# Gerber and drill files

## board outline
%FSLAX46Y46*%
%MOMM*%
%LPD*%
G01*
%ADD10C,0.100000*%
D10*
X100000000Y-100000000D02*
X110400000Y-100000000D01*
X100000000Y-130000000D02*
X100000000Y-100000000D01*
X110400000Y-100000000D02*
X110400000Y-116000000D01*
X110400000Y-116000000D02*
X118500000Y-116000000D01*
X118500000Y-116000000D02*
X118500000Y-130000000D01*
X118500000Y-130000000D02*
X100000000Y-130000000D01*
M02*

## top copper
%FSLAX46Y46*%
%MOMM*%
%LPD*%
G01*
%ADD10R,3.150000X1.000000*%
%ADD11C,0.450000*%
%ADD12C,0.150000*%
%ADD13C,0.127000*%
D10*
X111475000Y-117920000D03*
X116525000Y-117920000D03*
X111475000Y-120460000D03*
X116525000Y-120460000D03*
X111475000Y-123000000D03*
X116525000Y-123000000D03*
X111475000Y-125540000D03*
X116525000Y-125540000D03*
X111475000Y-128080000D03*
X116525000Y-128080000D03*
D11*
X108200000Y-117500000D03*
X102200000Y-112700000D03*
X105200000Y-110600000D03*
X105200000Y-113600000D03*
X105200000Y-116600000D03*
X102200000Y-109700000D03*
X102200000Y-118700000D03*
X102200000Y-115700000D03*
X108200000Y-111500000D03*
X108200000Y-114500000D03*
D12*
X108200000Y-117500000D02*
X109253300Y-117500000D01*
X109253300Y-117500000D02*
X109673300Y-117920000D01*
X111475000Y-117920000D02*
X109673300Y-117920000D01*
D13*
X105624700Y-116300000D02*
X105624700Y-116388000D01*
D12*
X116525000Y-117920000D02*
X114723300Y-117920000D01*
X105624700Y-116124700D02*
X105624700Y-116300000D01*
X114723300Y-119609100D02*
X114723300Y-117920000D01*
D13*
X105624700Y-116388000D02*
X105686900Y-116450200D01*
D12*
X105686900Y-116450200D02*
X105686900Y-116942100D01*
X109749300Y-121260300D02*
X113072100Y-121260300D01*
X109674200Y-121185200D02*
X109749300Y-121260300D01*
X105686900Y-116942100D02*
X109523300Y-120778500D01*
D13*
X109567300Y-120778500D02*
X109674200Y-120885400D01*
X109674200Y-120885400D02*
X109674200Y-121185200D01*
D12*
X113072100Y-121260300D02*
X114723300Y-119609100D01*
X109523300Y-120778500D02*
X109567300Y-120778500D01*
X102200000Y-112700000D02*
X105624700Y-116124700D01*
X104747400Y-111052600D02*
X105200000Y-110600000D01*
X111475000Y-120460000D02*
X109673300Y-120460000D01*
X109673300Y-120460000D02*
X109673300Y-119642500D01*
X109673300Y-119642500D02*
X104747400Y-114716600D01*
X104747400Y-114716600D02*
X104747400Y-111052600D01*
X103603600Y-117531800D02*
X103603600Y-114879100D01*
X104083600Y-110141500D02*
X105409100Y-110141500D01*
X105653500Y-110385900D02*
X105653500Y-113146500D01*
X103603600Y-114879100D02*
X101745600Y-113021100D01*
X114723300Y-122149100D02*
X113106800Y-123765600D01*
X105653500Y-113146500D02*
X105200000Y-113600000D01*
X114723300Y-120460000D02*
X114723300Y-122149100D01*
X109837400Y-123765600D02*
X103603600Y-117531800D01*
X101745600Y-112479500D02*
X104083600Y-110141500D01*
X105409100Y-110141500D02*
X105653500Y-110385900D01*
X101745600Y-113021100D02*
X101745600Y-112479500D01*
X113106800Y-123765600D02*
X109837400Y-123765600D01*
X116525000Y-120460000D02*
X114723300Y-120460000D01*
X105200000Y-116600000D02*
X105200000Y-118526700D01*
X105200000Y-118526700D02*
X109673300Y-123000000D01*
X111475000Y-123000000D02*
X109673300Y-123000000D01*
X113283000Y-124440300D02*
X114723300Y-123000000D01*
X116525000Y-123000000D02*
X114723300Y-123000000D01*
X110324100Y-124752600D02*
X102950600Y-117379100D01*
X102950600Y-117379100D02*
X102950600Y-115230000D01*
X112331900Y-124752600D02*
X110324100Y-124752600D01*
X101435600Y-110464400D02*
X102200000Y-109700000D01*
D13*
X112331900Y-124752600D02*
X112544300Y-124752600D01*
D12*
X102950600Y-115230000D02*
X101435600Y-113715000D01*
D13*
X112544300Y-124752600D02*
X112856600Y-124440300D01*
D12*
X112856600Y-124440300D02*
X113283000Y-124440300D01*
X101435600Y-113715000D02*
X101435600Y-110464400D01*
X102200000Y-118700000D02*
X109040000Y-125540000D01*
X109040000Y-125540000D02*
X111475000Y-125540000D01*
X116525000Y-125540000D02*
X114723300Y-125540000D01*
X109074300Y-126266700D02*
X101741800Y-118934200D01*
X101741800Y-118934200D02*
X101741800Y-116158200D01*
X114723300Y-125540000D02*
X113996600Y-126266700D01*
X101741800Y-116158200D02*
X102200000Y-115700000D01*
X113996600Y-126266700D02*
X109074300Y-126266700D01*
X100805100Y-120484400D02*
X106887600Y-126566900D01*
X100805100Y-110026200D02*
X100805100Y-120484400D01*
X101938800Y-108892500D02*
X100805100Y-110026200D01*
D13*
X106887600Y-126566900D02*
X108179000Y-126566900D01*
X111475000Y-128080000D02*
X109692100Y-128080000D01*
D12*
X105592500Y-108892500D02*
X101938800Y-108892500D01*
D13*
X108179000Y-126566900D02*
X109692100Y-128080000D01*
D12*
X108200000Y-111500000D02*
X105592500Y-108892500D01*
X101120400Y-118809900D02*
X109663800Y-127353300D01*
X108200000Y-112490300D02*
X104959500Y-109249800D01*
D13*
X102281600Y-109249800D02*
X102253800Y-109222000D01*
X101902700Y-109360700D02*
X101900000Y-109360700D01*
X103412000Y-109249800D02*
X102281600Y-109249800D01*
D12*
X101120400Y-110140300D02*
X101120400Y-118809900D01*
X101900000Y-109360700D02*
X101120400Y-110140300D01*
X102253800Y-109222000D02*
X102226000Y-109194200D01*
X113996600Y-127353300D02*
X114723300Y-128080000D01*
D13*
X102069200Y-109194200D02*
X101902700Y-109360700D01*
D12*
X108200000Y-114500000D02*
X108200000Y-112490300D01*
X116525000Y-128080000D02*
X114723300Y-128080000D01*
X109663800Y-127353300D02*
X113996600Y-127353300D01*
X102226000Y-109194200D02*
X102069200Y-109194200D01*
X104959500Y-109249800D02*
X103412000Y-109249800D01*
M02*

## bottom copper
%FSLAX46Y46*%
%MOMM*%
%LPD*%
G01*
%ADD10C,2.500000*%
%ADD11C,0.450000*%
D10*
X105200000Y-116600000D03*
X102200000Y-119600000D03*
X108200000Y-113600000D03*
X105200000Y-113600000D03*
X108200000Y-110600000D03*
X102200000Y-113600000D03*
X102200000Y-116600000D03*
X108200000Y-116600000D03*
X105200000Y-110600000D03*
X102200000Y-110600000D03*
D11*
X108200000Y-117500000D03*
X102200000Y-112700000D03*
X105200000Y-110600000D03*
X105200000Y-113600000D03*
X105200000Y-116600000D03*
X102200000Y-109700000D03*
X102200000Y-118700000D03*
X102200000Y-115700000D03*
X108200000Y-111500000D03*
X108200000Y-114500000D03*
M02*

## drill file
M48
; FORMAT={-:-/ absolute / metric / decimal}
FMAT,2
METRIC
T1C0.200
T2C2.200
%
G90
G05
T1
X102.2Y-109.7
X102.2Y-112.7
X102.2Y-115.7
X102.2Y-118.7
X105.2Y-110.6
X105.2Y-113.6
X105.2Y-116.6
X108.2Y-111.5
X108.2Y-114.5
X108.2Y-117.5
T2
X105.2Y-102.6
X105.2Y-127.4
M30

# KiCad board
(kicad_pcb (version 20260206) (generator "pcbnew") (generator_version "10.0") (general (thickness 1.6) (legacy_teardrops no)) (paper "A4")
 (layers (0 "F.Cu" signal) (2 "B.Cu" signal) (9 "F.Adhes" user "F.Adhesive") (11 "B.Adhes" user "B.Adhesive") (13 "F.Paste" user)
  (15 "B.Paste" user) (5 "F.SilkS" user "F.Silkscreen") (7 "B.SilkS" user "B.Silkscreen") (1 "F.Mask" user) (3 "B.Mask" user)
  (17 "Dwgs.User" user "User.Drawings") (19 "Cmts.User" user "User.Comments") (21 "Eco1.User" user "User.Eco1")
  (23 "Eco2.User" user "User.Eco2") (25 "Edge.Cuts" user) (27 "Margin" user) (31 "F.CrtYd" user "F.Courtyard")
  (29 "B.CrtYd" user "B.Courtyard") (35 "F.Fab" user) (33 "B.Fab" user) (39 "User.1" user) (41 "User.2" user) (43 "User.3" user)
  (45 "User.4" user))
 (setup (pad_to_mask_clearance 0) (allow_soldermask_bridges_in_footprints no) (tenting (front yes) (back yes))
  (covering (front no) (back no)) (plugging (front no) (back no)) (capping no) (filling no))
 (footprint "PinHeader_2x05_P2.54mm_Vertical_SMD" (layer "F.Cu") (at 114 123)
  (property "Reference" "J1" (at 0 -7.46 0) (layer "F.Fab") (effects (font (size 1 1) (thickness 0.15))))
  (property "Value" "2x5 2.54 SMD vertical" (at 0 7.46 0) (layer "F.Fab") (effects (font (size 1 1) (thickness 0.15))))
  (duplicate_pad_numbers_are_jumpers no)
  (pad "1" smd rect (at -2.525 -5.08) (size 3.15 1) (layers "F.Cu" "F.Mask" "F.Paste") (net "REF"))
  (pad "2" smd rect (at 2.525 -5.08) (size 3.15 1) (layers "F.Cu" "F.Mask" "F.Paste") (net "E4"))
  (pad "3" smd rect (at -2.525 -2.54) (size 3.15 1) (layers "F.Cu" "F.Mask" "F.Paste") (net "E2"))
  (pad "4" smd rect (at 2.525 -2.54) (size 3.15 1) (layers "F.Cu" "F.Mask" "F.Paste") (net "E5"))
  (pad "5" smd rect (at -2.525 0) (size 3.15 1) (layers "F.Cu" "F.Mask" "F.Paste") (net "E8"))
  (pad "6" smd rect (at 2.525 0) (size 3.15 1) (layers "F.Cu" "F.Mask" "F.Paste") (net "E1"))
  (pad "7" smd rect (at -2.525 2.54) (size 3.15 1) (layers "F.Cu" "F.Mask" "F.Paste") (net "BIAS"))
  (pad "8" smd rect (at 2.525 2.54) (size 3.15 1) (layers "F.Cu" "F.Mask" "F.Paste") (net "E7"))
  (pad "9" smd rect (at -2.525 5.08) (size 3.15 1) (layers "F.Cu" "F.Mask" "F.Paste") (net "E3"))
  (pad "10" smd rect (at 2.525 5.08) (size 3.15 1) (layers "F.Cu" "F.Mask" "F.Paste") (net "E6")))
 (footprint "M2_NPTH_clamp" (layer "F.Cu") (at 105.2 127.4)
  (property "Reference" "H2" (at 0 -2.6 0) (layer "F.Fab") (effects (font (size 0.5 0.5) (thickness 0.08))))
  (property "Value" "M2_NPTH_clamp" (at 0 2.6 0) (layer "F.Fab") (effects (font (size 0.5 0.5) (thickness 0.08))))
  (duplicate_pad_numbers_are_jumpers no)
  (pad "" np_thru_hole circle (at 0 0) (size 2.2 2.2) (drill 2.2) (layers "*.Cu" "*.Mask")))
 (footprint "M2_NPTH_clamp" (layer "F.Cu") (at 105.2 102.6)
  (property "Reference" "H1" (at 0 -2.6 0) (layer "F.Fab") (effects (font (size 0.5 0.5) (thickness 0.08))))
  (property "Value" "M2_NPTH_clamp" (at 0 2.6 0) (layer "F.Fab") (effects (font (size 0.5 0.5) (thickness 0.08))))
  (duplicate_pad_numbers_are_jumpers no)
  (pad "" np_thru_hole circle (at 0 0) (size 2.2 2.2) (drill 2.2) (layers "*.Cu" "*.Mask")))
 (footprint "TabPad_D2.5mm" (layer "B.Cu") (at 105.2 116.6 180)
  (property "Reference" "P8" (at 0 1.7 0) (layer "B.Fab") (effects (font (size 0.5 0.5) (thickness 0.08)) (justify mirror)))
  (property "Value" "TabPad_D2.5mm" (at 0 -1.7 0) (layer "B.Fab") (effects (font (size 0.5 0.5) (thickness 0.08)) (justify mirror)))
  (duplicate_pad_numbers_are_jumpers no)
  (pad "1" smd circle (at 0 0 180) (size 2.5 2.5) (layers "B.Cu" "B.Mask") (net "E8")))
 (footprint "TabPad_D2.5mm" (layer "B.Cu") (at 102.2 119.6 180)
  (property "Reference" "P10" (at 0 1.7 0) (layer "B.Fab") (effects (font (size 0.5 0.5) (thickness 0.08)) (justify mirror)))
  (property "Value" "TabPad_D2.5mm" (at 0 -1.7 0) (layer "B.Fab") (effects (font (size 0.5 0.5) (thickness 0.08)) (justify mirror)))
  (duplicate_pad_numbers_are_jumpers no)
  (pad "1" smd circle (at 0 0 180) (size 2.5 2.5) (layers "B.Cu" "B.Mask") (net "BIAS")))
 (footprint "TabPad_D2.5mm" (layer "B.Cu") (at 108.2 113.6 180)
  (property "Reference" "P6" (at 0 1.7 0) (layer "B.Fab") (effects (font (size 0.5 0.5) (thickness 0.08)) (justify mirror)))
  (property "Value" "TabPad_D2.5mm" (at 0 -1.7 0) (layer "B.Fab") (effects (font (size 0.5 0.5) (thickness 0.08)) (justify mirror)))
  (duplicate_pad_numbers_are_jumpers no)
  (pad "1" smd circle (at 0 0 180) (size 2.5 2.5) (layers "B.Cu" "B.Mask") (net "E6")))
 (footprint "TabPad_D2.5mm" (layer "B.Cu") (at 105.2 113.6 180)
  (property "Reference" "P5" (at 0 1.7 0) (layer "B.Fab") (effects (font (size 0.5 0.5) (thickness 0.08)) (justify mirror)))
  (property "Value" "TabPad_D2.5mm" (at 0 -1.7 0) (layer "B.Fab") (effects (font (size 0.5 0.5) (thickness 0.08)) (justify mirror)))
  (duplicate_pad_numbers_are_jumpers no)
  (pad "1" smd circle (at 0 0 180) (size 2.5 2.5) (layers "B.Cu" "B.Mask") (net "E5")))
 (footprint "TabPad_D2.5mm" (layer "B.Cu") (at 108.2 110.6 180)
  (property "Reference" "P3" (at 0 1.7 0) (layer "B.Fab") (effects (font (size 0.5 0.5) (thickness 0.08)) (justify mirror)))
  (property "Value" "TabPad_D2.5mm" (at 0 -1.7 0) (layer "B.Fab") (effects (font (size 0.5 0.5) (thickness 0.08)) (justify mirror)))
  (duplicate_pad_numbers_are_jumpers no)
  (pad "1" smd circle (at 0 0 180) (size 2.5 2.5) (layers "B.Cu" "B.Mask") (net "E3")))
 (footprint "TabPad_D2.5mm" (layer "B.Cu") (at 102.2 113.6 180)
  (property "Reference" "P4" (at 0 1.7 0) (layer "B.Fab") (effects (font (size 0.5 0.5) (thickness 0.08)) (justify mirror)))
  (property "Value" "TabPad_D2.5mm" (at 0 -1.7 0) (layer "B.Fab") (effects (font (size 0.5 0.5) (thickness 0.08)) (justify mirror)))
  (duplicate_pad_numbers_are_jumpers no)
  (pad "1" smd circle (at 0 0 180) (size 2.5 2.5) (layers "B.Cu" "B.Mask") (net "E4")))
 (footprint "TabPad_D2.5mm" (layer "B.Cu") (at 102.2 116.6 180)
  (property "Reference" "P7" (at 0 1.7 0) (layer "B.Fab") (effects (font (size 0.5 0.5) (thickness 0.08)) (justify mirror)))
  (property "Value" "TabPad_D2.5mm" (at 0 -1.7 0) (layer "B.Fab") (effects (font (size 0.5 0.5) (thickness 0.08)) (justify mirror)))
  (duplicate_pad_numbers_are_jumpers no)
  (pad "1" smd circle (at 0 0 180) (size 2.5 2.5) (layers "B.Cu" "B.Mask") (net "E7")))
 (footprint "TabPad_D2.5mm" (layer "B.Cu") (at 108.2 116.6 180)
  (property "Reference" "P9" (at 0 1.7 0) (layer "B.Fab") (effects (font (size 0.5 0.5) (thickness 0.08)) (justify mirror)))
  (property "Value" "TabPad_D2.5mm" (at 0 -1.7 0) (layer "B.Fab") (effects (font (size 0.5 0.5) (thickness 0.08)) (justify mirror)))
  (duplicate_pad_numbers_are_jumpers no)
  (pad "1" smd circle (at 0 0 180) (size 2.5 2.5) (layers "B.Cu" "B.Mask") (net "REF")))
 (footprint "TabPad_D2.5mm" (layer "B.Cu") (at 105.2 110.6 180)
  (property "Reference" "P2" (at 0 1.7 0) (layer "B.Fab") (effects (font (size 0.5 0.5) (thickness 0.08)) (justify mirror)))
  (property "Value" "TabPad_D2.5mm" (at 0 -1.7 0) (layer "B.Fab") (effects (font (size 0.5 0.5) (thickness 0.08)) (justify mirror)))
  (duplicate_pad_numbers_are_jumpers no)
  (pad "1" smd circle (at 0 0 180) (size 2.5 2.5) (layers "B.Cu" "B.Mask") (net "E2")))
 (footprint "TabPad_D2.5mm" (layer "B.Cu") (at 102.2 110.6 180)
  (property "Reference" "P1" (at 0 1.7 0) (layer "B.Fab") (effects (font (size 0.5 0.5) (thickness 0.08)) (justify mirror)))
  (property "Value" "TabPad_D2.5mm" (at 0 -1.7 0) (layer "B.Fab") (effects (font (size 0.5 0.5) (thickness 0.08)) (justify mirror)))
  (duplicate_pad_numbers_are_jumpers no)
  (pad "1" smd circle (at 0 0 180) (size 2.5 2.5) (layers "B.Cu" "B.Mask") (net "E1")))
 (gr_line (start 100 100) (end 110.4 100) (stroke (width 0.1) (type default)) (layer "Edge.Cuts"))
 (gr_line (start 100 130) (end 100 100) (stroke (width 0.1) (type default)) (layer "Edge.Cuts"))
 (gr_line (start 110.4 100) (end 110.4 116) (stroke (width 0.1) (type default)) (layer "Edge.Cuts"))
 (gr_line (start 110.4 116) (end 118.5 116) (stroke (width 0.1) (type default)) (layer "Edge.Cuts"))
 (gr_line (start 118.5 116) (end 118.5 130) (stroke (width 0.1) (type default)) (layer "Edge.Cuts"))
 (gr_line (start 118.5 130) (end 100 130) (stroke (width 0.1) (type default)) (layer "Edge.Cuts"))
 (segment (start 108.2 117.5) (end 109.2533 117.5) (width 0.15) (layer "F.Cu") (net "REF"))
 (segment (start 109.2533 117.5) (end 109.6733 117.92) (width 0.15) (layer "F.Cu") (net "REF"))
 (segment (start 111.475 117.92) (end 109.6733 117.92) (width 0.15) (layer "F.Cu") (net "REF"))
 (via (at 108.2 117.5) (size 0.45) (drill 0.2) (layers "F.Cu" "B.Cu") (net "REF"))
 (segment (start 105.6247 116.3) (end 105.6247 116.388) (width 0.127) (layer "F.Cu") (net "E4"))
 (segment (start 116.525 117.92) (end 114.7233 117.92) (width 0.15) (layer "F.Cu") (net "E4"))
 (segment (start 105.6247 116.1247) (end 105.6247 116.3) (width 0.15) (layer "F.Cu") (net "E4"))
 (segment (start 114.7233 119.6091) (end 114.7233 117.92) (width 0.15) (layer "F.Cu") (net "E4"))
 (segment (start 105.6247 116.388) (end 105.6869 116.4502) (width 0.127) (layer "F.Cu") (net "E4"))
 (segment (start 105.6869 116.4502) (end 105.6869 116.9421) (width 0.15) (layer "F.Cu") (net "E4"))
 (segment (start 109.7493 121.2603) (end 113.0721 121.2603) (width 0.15) (layer "F.Cu") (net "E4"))
 (segment (start 109.6742 121.1852) (end 109.7493 121.2603) (width 0.15) (layer "F.Cu") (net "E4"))
 (segment (start 105.6869 116.9421) (end 109.5233 120.7785) (width 0.15) (layer "F.Cu") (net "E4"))
 (segment (start 109.5673 120.7785) (end 109.6742 120.8854) (width 0.127) (layer "F.Cu") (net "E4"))
 (segment (start 109.6742 120.8854) (end 109.6742 121.1852) (width 0.127) (layer "F.Cu") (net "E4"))
 (segment (start 113.0721 121.2603) (end 114.7233 119.6091) (width 0.15) (layer "F.Cu") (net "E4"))
 (segment (start 109.5233 120.7785) (end 109.5673 120.7785) (width 0.15) (layer "F.Cu") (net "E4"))
 (segment (start 102.2 112.7) (end 105.6247 116.1247) (width 0.15) (layer "F.Cu") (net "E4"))
 (via (at 102.2 112.7) (size 0.45) (drill 0.2) (layers "F.Cu" "B.Cu") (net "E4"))
 (segment (start 104.7474 111.0526) (end 105.2 110.6) (width 0.15) (layer "F.Cu") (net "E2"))
 (segment (start 111.475 120.46) (end 109.6733 120.46) (width 0.15) (layer "F.Cu") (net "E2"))
 (segment (start 109.6733 120.46) (end 109.6733 119.6425) (width 0.15) (layer "F.Cu") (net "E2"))
 (segment (start 109.6733 119.6425) (end 104.7474 114.7166) (width 0.15) (layer "F.Cu") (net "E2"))
 (segment (start 104.7474 114.7166) (end 104.7474 111.0526) (width 0.15) (layer "F.Cu") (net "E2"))
 (via (at 105.2 110.6) (size 0.45) (drill 0.2) (layers "F.Cu" "B.Cu") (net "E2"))
 (segment (start 103.6036 117.5318) (end 103.6036 114.8791) (width 0.15) (layer "F.Cu") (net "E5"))
 (segment (start 104.0836 110.1415) (end 105.4091 110.1415) (width 0.15) (layer "F.Cu") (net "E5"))
 (segment (start 105.6535 110.3859) (end 105.6535 113.1465) (width 0.15) (layer "F.Cu") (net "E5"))
 (segment (start 103.6036 114.8791) (end 101.7456 113.0211) (width 0.15) (layer "F.Cu") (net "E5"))
 (segment (start 114.7233 122.1491) (end 113.1068 123.7656) (width 0.15) (layer "F.Cu") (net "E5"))
 (segment (start 105.6535 113.1465) (end 105.2 113.6) (width 0.15) (layer "F.Cu") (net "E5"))
 (segment (start 114.7233 120.46) (end 114.7233 122.1491) (width 0.15) (layer "F.Cu") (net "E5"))
 (segment (start 109.8374 123.7656) (end 103.6036 117.5318) (width 0.15) (layer "F.Cu") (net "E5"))
 (segment (start 101.7456 112.4795) (end 104.0836 110.1415) (width 0.15) (layer "F.Cu") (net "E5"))
 (segment (start 105.4091 110.1415) (end 105.6535 110.3859) (width 0.15) (layer "F.Cu") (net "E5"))
 (segment (start 101.7456 113.0211) (end 101.7456 112.4795) (width 0.15) (layer "F.Cu") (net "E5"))
 (segment (start 113.1068 123.7656) (end 109.8374 123.7656) (width 0.15) (layer "F.Cu") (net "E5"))
 (segment (start 116.525 120.46) (end 114.7233 120.46) (width 0.15) (layer "F.Cu") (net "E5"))
 (via (at 105.2 113.6) (size 0.45) (drill 0.2) (layers "F.Cu" "B.Cu") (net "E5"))
 (segment (start 105.2 116.6) (end 105.2 118.5267) (width 0.15) (layer "F.Cu") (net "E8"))
 (segment (start 105.2 118.5267) (end 109.6733 123) (width 0.15) (layer "F.Cu") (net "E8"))
 (segment (start 111.475 123) (end 109.6733 123) (width 0.15) (layer "F.Cu") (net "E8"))
 (via (at 105.2 116.6) (size 0.45) (drill 0.2) (layers "F.Cu" "B.Cu") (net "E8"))
 (segment (start 113.283 124.4403) (end 114.7233 123) (width 0.15) (layer "F.Cu") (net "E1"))
 (segment (start 116.525 123) (end 114.7233 123) (width 0.15) (layer "F.Cu") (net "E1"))
 (segment (start 110.3241 124.7526) (end 102.9506 117.3791) (width 0.15) (layer "F.Cu") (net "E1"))
 (segment (start 102.9506 117.3791) (end 102.9506 115.23) (width 0.15) (layer "F.Cu") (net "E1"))
 (segment (start 112.3319 124.7526) (end 110.3241 124.7526) (width 0.15) (layer "F.Cu") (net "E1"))
 (segment (start 101.4356 110.4644) (end 102.2 109.7) (width 0.15) (layer "F.Cu") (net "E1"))
 (segment (start 112.3319 124.7526) (end 112.5443 124.7526) (width 0.127) (layer "F.Cu") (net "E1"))
 (segment (start 102.9506 115.23) (end 101.4356 113.715) (width 0.15) (layer "F.Cu") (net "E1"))
 (segment (start 112.5443 124.7526) (end 112.8566 124.4403) (width 0.127) (layer "F.Cu") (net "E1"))
 (segment (start 112.8566 124.4403) (end 113.283 124.4403) (width 0.15) (layer "F.Cu") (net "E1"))
 (segment (start 101.4356 113.715) (end 101.4356 110.4644) (width 0.15) (layer "F.Cu") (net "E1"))
 (via (at 102.2 109.7) (size 0.45) (drill 0.2) (layers "F.Cu" "B.Cu") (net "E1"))
 (segment (start 102.2 118.7) (end 109.04 125.54) (width 0.15) (layer "F.Cu") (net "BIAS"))
 (segment (start 109.04 125.54) (end 111.475 125.54) (width 0.15) (layer "F.Cu") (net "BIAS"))
 (via (at 102.2 118.7) (size 0.45) (drill 0.2) (layers "F.Cu" "B.Cu") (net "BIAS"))
 (segment (start 116.525 125.54) (end 114.7233 125.54) (width 0.15) (layer "F.Cu") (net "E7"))
 (segment (start 109.0743 126.2667) (end 101.7418 118.9342) (width 0.15) (layer "F.Cu") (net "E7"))
 (segment (start 101.7418 118.9342) (end 101.7418 116.1582) (width 0.15) (layer "F.Cu") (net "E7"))
 (segment (start 114.7233 125.54) (end 113.9966 126.2667) (width 0.15) (layer "F.Cu") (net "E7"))
 (segment (start 101.7418 116.1582) (end 102.2 115.7) (width 0.15) (layer "F.Cu") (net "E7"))
 (segment (start 113.9966 126.2667) (end 109.0743 126.2667) (width 0.15) (layer "F.Cu") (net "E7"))
 (via (at 102.2 115.7) (size 0.45) (drill 0.2) (layers "F.Cu" "B.Cu") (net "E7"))
 (segment (start 100.8051 120.4844) (end 106.8876 126.5669) (width 0.15) (layer "F.Cu") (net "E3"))
 (segment (start 100.8051 110.0262) (end 100.8051 120.4844) (width 0.15) (layer "F.Cu") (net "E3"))
 (segment (start 101.9388 108.8925) (end 100.8051 110.0262) (width 0.15) (layer "F.Cu") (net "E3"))
 (segment (start 106.8876 126.5669) (end 108.179 126.5669) (width 0.127) (layer "F.Cu") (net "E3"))
 (segment (start 111.475 128.08) (end 109.6921 128.08) (width 0.127) (layer "F.Cu") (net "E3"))
 (segment (start 105.5925 108.8925) (end 101.9388 108.8925) (width 0.15) (layer "F.Cu") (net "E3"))
 (segment (start 108.179 126.5669) (end 109.6921 128.08) (width 0.127) (layer "F.Cu") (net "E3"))
 (segment (start 108.2 111.5) (end 105.5925 108.8925) (width 0.15) (layer "F.Cu") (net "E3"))
 (via (at 108.2 111.5) (size 0.45) (drill 0.2) (layers "F.Cu" "B.Cu") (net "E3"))
 (segment (start 101.1204 118.8099) (end 109.6638 127.3533) (width 0.15) (layer "F.Cu") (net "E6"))
 (segment (start 108.2 112.4903) (end 104.9595 109.2498) (width 0.15) (layer "F.Cu") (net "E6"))
 (segment (start 102.2816 109.2498) (end 102.2538 109.222) (width 0.127) (layer "F.Cu") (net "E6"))
 (segment (start 101.9027 109.3607) (end 101.9 109.3607) (width 0.127) (layer "F.Cu") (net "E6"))
 (segment (start 103.412 109.2498) (end 102.2816 109.2498) (width 0.127) (layer "F.Cu") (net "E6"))
 (segment (start 101.1204 110.1403) (end 101.1204 118.8099) (width 0.15) (layer "F.Cu") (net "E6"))
 (segment (start 101.9 109.3607) (end 101.1204 110.1403) (width 0.15) (layer "F.Cu") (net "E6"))
 (segment (start 102.2538 109.222) (end 102.226 109.1942) (width 0.15) (layer "F.Cu") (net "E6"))
 (segment (start 113.9966 127.3533) (end 114.7233 128.08) (width 0.15) (layer "F.Cu") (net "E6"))
 (segment (start 102.0692 109.1942) (end 101.9027 109.3607) (width 0.127) (layer "F.Cu") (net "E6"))
 (segment (start 108.2 114.5) (end 108.2 112.4903) (width 0.15) (layer "F.Cu") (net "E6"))
 (segment (start 116.525 128.08) (end 114.7233 128.08) (width 0.15) (layer "F.Cu") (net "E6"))
 (segment (start 109.6638 127.3533) (end 113.9966 127.3533) (width 0.15) (layer "F.Cu") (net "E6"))
 (segment (start 102.226 109.1942) (end 102.0692 109.1942) (width 0.15) (layer "F.Cu") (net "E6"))
 (segment (start 104.9595 109.2498) (end 103.412 109.2498) (width 0.15) (layer "F.Cu") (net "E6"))
 (via (at 108.2 114.5) (size 0.45) (drill 0.2) (layers "F.Cu" "B.Cu") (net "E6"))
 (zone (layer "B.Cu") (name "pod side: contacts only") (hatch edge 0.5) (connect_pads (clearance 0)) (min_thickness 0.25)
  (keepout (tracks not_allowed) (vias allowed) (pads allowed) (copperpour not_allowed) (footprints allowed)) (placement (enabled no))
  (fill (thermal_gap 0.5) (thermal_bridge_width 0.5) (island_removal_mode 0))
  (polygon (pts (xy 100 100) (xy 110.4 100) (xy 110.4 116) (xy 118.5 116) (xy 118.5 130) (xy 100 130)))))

